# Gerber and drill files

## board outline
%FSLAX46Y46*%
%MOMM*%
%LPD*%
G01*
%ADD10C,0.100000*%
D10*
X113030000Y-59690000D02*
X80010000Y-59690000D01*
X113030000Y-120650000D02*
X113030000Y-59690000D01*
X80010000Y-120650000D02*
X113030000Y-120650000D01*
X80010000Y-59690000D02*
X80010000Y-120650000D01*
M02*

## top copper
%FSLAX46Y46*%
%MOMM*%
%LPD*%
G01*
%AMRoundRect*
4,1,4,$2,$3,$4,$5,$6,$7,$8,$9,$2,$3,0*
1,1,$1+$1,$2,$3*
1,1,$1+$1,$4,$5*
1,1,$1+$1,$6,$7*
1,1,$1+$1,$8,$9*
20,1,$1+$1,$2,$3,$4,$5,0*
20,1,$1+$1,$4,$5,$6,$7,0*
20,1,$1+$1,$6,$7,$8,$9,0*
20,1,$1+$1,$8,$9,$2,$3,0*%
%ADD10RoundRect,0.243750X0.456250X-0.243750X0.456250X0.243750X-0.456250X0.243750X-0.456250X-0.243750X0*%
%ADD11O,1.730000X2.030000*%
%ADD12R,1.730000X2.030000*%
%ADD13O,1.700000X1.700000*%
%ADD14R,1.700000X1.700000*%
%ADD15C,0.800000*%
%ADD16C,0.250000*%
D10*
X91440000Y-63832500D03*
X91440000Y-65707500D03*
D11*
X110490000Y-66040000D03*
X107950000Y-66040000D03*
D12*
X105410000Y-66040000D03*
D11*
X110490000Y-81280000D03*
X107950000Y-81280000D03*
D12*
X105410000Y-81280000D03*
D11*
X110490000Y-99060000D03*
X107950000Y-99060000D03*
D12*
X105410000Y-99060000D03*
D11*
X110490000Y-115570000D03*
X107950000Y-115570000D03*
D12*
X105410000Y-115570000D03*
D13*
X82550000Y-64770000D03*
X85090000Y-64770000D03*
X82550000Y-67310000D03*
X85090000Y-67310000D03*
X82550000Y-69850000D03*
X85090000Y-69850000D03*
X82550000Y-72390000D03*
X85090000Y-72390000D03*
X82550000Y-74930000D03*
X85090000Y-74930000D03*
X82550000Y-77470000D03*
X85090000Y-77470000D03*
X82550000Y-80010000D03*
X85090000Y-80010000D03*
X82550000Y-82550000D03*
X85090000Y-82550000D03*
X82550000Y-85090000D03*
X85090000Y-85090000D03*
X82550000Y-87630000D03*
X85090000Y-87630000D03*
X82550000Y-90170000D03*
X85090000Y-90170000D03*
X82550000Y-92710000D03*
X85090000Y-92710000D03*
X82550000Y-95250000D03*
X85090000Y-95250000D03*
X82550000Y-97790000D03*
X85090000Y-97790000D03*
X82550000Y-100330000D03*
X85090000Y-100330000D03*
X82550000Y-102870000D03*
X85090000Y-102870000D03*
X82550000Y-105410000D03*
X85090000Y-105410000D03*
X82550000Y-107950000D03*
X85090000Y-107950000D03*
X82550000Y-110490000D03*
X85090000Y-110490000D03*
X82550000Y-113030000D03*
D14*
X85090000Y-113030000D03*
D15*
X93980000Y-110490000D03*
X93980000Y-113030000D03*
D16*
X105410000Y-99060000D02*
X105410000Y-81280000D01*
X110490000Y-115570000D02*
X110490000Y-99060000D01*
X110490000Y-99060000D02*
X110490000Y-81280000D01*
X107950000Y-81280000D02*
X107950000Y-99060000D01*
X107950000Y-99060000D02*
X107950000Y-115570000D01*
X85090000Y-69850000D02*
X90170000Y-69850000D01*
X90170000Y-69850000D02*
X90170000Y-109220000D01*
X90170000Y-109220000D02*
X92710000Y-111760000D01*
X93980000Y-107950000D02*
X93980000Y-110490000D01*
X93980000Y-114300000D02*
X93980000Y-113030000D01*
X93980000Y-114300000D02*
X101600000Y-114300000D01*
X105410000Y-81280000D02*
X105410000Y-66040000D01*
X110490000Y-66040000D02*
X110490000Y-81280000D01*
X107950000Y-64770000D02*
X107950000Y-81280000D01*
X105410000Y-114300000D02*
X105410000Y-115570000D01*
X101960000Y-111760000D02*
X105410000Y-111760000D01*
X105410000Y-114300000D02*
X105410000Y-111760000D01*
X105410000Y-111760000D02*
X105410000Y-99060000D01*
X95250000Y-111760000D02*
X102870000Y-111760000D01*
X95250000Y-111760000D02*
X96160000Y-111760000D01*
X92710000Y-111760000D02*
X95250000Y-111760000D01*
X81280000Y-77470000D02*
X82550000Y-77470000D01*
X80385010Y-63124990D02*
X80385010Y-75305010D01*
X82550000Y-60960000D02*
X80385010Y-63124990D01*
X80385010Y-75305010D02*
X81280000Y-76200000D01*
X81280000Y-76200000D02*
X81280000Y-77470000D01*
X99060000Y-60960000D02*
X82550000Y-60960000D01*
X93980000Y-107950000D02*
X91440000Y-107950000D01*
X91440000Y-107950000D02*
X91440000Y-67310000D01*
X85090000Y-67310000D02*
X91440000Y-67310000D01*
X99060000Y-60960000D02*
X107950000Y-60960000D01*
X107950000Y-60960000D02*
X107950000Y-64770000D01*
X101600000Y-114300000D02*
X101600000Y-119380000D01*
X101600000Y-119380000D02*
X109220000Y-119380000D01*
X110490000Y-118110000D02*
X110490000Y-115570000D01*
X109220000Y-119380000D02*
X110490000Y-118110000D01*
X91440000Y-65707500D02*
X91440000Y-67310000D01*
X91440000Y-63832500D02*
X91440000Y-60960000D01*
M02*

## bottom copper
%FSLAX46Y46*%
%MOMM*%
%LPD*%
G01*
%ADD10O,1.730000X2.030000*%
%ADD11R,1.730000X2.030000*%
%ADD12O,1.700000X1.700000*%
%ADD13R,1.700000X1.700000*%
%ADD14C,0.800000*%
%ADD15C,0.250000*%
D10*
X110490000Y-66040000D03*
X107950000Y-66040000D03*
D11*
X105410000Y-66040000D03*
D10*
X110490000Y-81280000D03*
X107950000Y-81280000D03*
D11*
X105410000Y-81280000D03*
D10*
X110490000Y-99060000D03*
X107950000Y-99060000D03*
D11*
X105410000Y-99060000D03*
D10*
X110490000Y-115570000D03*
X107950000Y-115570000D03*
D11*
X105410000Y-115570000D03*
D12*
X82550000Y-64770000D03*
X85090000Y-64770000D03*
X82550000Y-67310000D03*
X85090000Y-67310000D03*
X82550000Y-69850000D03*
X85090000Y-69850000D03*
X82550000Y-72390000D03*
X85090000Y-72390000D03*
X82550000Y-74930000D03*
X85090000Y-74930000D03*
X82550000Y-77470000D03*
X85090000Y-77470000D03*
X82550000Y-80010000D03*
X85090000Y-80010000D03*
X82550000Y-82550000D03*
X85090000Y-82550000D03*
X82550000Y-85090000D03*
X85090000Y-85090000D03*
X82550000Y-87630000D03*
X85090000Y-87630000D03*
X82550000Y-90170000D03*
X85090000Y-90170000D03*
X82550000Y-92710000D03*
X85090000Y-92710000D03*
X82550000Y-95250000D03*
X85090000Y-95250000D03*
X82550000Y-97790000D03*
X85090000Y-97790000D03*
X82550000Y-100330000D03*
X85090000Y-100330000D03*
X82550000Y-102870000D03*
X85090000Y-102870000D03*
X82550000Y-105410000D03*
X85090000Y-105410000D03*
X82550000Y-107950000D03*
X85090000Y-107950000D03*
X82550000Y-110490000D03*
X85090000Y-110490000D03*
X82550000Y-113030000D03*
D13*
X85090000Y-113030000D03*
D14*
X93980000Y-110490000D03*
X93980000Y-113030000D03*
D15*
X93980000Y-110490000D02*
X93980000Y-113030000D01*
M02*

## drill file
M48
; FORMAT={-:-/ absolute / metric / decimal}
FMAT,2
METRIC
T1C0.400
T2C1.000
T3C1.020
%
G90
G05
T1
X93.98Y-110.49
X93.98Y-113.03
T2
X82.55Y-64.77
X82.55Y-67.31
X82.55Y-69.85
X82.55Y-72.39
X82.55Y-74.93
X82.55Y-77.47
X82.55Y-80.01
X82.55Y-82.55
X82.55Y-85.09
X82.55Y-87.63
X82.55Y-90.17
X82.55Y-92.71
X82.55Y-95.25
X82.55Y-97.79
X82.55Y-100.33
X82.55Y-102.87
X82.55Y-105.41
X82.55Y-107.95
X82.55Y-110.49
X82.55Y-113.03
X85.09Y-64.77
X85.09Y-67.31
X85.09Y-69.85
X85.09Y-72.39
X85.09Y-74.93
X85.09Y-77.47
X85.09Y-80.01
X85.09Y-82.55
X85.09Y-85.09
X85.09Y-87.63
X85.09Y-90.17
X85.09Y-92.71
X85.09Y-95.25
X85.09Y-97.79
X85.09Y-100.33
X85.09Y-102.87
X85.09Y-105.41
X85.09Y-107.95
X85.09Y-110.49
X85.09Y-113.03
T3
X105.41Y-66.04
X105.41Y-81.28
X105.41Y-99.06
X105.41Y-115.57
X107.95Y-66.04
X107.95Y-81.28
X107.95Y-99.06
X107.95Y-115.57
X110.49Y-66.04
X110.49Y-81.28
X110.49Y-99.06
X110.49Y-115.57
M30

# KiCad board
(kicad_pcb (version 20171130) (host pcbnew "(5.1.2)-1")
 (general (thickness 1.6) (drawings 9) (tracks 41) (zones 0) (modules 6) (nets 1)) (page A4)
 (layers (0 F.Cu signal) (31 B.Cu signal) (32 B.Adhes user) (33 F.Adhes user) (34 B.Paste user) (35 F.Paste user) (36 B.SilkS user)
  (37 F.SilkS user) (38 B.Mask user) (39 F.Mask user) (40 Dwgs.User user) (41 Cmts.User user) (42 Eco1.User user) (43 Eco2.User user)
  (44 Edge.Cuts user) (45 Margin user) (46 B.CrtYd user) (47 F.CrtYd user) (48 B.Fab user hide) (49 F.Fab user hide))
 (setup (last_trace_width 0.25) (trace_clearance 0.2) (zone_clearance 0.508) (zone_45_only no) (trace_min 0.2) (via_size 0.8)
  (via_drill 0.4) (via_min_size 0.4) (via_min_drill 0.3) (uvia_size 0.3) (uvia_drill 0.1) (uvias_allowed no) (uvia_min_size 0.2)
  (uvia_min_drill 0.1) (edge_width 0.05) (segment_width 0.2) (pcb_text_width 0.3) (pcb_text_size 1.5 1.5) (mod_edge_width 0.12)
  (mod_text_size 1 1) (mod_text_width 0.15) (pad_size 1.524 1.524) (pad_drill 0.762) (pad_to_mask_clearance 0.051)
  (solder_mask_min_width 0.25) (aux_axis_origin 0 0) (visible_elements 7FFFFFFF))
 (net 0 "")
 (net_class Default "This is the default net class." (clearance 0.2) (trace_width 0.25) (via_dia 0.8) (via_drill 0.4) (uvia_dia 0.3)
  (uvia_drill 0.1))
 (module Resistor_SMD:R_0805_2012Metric (layer F.Cu) (at 91.44 64.77 90)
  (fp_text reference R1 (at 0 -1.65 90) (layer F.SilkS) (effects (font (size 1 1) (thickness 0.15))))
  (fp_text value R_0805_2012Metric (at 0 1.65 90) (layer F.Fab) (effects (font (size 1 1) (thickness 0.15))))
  (pad 2 smd roundrect (at 0.9375 0 90) (size 0.975 1.4) (layers F.Cu F.Paste F.Mask) (roundrect_rratio 0.25))
  (pad 1 smd roundrect (at -0.9375 0 90) (size 0.975 1.4) (layers F.Cu F.Paste F.Mask) (roundrect_rratio 0.25)))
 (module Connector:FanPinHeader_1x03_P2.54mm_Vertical (layer F.Cu) (at 105.41 66.04)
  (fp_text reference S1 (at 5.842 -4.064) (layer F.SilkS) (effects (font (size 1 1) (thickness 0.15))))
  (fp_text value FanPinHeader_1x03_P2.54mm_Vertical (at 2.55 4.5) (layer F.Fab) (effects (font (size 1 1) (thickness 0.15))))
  (pad 3 thru_hole oval (at 5.08 0 90) (size 2.03 1.73) (drill 1.02) (layers *.Cu *.Mask))
  (pad 2 thru_hole oval (at 2.54 0 90) (size 2.03 1.73) (drill 1.02) (layers *.Cu *.Mask))
  (pad 1 thru_hole rect (at 0 0 90) (size 2.03 1.73) (drill 1.02) (layers *.Cu *.Mask)))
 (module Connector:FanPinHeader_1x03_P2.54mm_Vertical (layer F.Cu) (at 105.41 81.28)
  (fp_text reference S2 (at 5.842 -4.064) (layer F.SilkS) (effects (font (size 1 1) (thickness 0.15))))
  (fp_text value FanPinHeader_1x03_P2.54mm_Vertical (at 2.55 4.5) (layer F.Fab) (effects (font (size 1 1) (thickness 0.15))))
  (pad 3 thru_hole oval (at 5.08 0 90) (size 2.03 1.73) (drill 1.02) (layers *.Cu *.Mask))
  (pad 2 thru_hole oval (at 2.54 0 90) (size 2.03 1.73) (drill 1.02) (layers *.Cu *.Mask))
  (pad 1 thru_hole rect (at 0 0 90) (size 2.03 1.73) (drill 1.02) (layers *.Cu *.Mask)))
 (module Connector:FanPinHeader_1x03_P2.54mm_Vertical (layer F.Cu) (at 105.41 99.06)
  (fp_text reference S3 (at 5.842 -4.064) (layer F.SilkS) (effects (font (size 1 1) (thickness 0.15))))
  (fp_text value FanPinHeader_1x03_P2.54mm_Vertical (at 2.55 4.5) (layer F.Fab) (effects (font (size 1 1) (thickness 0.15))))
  (pad 3 thru_hole oval (at 5.08 0 90) (size 2.03 1.73) (drill 1.02) (layers *.Cu *.Mask))
  (pad 2 thru_hole oval (at 2.54 0 90) (size 2.03 1.73) (drill 1.02) (layers *.Cu *.Mask))
  (pad 1 thru_hole rect (at 0 0 90) (size 2.03 1.73) (drill 1.02) (layers *.Cu *.Mask)))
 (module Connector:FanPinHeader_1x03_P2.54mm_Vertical (layer F.Cu) (at 105.41 115.57)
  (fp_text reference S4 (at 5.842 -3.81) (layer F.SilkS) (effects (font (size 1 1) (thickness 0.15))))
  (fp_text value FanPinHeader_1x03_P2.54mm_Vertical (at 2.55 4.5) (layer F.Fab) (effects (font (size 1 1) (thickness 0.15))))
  (pad 3 thru_hole oval (at 5.08 0 90) (size 2.03 1.73) (drill 1.02) (layers *.Cu *.Mask))
  (pad 2 thru_hole oval (at 2.54 0 90) (size 2.03 1.73) (drill 1.02) (layers *.Cu *.Mask))
  (pad 1 thru_hole rect (at 0 0 90) (size 2.03 1.73) (drill 1.02) (layers *.Cu *.Mask)))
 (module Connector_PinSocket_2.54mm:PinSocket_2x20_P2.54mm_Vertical (layer B.Cu) (at 85.09 113.03)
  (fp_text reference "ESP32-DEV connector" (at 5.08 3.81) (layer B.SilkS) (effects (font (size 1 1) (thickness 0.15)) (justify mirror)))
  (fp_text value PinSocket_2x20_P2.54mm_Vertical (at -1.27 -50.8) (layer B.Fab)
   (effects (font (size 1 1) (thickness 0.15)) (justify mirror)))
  (pad 40 thru_hole oval (at -2.54 -48.26) (size 1.7 1.7) (drill 1) (layers *.Cu *.Mask))
  (pad 39 thru_hole oval (at 0 -48.26) (size 1.7 1.7) (drill 1) (layers *.Cu *.Mask))
  (pad 38 thru_hole oval (at -2.54 -45.72) (size 1.7 1.7) (drill 1) (layers *.Cu *.Mask))
  (pad 37 thru_hole oval (at 0 -45.72) (size 1.7 1.7) (drill 1) (layers *.Cu *.Mask))
  (pad 36 thru_hole oval (at -2.54 -43.18) (size 1.7 1.7) (drill 1) (layers *.Cu *.Mask))
  (pad 35 thru_hole oval (at 0 -43.18) (size 1.7 1.7) (drill 1) (layers *.Cu *.Mask))
  (pad 34 thru_hole oval (at -2.54 -40.64) (size 1.7 1.7) (drill 1) (layers *.Cu *.Mask))
  (pad 33 thru_hole oval (at 0 -40.64) (size 1.7 1.7) (drill 1) (layers *.Cu *.Mask))
  (pad 32 thru_hole oval (at -2.54 -38.1) (size 1.7 1.7) (drill 1) (layers *.Cu *.Mask))
  (pad 31 thru_hole oval (at 0 -38.1) (size 1.7 1.7) (drill 1) (layers *.Cu *.Mask))
  (pad 30 thru_hole oval (at -2.54 -35.56) (size 1.7 1.7) (drill 1) (layers *.Cu *.Mask))
  (pad 29 thru_hole oval (at 0 -35.56) (size 1.7 1.7) (drill 1) (layers *.Cu *.Mask))
  (pad 28 thru_hole oval (at -2.54 -33.02) (size 1.7 1.7) (drill 1) (layers *.Cu *.Mask))
  (pad 27 thru_hole oval (at 0 -33.02) (size 1.7 1.7) (drill 1) (layers *.Cu *.Mask))
  (pad 26 thru_hole oval (at -2.54 -30.48) (size 1.7 1.7) (drill 1) (layers *.Cu *.Mask))
  (pad 25 thru_hole oval (at 0 -30.48) (size 1.7 1.7) (drill 1) (layers *.Cu *.Mask))
  (pad 24 thru_hole oval (at -2.54 -27.94) (size 1.7 1.7) (drill 1) (layers *.Cu *.Mask))
  (pad 23 thru_hole oval (at 0 -27.94) (size 1.7 1.7) (drill 1) (layers *.Cu *.Mask))
  (pad 22 thru_hole oval (at -2.54 -25.4) (size 1.7 1.7) (drill 1) (layers *.Cu *.Mask))
  (pad 21 thru_hole oval (at 0 -25.4) (size 1.7 1.7) (drill 1) (layers *.Cu *.Mask))
  (pad 20 thru_hole oval (at -2.54 -22.86) (size 1.7 1.7) (drill 1) (layers *.Cu *.Mask))
  (pad 19 thru_hole oval (at 0 -22.86) (size 1.7 1.7) (drill 1) (layers *.Cu *.Mask))
  (pad 18 thru_hole oval (at -2.54 -20.32) (size 1.7 1.7) (drill 1) (layers *.Cu *.Mask))
  (pad 17 thru_hole oval (at 0 -20.32) (size 1.7 1.7) (drill 1) (layers *.Cu *.Mask))
  (pad 16 thru_hole oval (at -2.54 -17.78) (size 1.7 1.7) (drill 1) (layers *.Cu *.Mask))
  (pad 15 thru_hole oval (at 0 -17.78) (size 1.7 1.7) (drill 1) (layers *.Cu *.Mask))
  (pad 14 thru_hole oval (at -2.54 -15.24) (size 1.7 1.7) (drill 1) (layers *.Cu *.Mask))
  (pad 13 thru_hole oval (at 0 -15.24) (size 1.7 1.7) (drill 1) (layers *.Cu *.Mask))
  (pad 12 thru_hole oval (at -2.54 -12.7) (size 1.7 1.7) (drill 1) (layers *.Cu *.Mask))
  (pad 11 thru_hole oval (at 0 -12.7) (size 1.7 1.7) (drill 1) (layers *.Cu *.Mask))
  (pad 10 thru_hole oval (at -2.54 -10.16) (size 1.7 1.7) (drill 1) (layers *.Cu *.Mask))
  (pad 9 thru_hole oval (at 0 -10.16) (size 1.7 1.7) (drill 1) (layers *.Cu *.Mask))
  (pad 8 thru_hole oval (at -2.54 -7.62) (size 1.7 1.7) (drill 1) (layers *.Cu *.Mask))
  (pad 7 thru_hole oval (at 0 -7.62) (size 1.7 1.7) (drill 1) (layers *.Cu *.Mask))
  (pad 6 thru_hole oval (at -2.54 -5.08) (size 1.7 1.7) (drill 1) (layers *.Cu *.Mask))
  (pad 5 thru_hole oval (at 0 -5.08) (size 1.7 1.7) (drill 1) (layers *.Cu *.Mask))
  (pad 4 thru_hole oval (at -2.54 -2.54) (size 1.7 1.7) (drill 1) (layers *.Cu *.Mask))
  (pad 3 thru_hole oval (at 0 -2.54) (size 1.7 1.7) (drill 1) (layers *.Cu *.Mask))
  (pad 2 thru_hole oval (at -2.54 0) (size 1.7 1.7) (drill 1) (layers *.Cu *.Mask))
  (pad 1 thru_hole rect (at 0 0) (size 1.7 1.7) (drill 1) (layers *.Cu *.Mask)))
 (gr_line (start 113.03 59.69) (end 80.01 59.69) (layer Edge.Cuts) (width 0.1))
 (gr_line (start 113.03 120.65) (end 113.03 59.69) (layer Edge.Cuts) (width 0.1))
 (gr_line (start 80.01 120.65) (end 113.03 120.65) (layer Edge.Cuts) (width 0.1))
 (gr_line (start 80.01 59.69) (end 80.01 120.65) (layer Edge.Cuts) (width 0.1))
 (segment (start 105.41 99.06) (end 105.41 81.28) (width 0.25) (layer F.Cu) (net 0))
 (segment (start 110.49 115.57) (end 110.49 99.06) (width 0.25) (layer F.Cu) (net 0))
 (segment (start 110.49 99.06) (end 110.49 81.28) (width 0.25) (layer F.Cu) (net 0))
 (segment (start 107.95 81.28) (end 107.95 99.06) (width 0.25) (layer F.Cu) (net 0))
 (segment (start 107.95 99.06) (end 107.95 115.57) (width 0.25) (layer F.Cu) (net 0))
 (segment (start 85.09 69.85) (end 90.17 69.85) (width 0.25) (layer F.Cu) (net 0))
 (segment (start 90.17 69.85) (end 90.17 109.22) (width 0.25) (layer F.Cu) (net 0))
 (segment (start 90.17 109.22) (end 92.71 111.76) (width 0.25) (layer F.Cu) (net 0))
 (segment (start 93.98 107.95) (end 93.98 110.49) (width 0.25) (layer F.Cu) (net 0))
 (via (at 93.98 110.49) (size 0.8) (drill 0.4) (layers F.Cu B.Cu) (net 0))
 (segment (start 93.98 114.3) (end 93.98 113.03) (width 0.25) (layer F.Cu) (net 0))
 (via (at 93.98 113.03) (size 0.8) (drill 0.4) (layers F.Cu B.Cu) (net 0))
 (segment (start 93.98 114.3) (end 101.6 114.3) (width 0.25) (layer F.Cu) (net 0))
 (segment (start 93.98 110.49) (end 93.98 113.03) (width 0.25) (layer B.Cu) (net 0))
 (segment (start 105.41 81.28) (end 105.41 66.04) (width 0.25) (layer F.Cu) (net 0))
 (segment (start 110.49 66.04) (end 110.49 81.28) (width 0.25) (layer F.Cu) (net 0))
 (segment (start 107.95 64.77) (end 107.95 81.28) (width 0.25) (layer F.Cu) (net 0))
 (segment (start 105.41 114.3) (end 105.41 115.57) (width 0.25) (layer F.Cu) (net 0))
 (segment (start 101.96 111.76) (end 105.41 111.76) (width 0.25) (layer F.Cu) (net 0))
 (segment (start 105.41 114.3) (end 105.41 111.76) (width 0.25) (layer F.Cu) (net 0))
 (segment (start 105.41 111.76) (end 105.41 99.06) (width 0.25) (layer F.Cu) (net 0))
 (segment (start 95.25 111.76) (end 102.87 111.76) (width 0.25) (layer F.Cu) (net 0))
 (segment (start 95.25 111.76) (end 96.16 111.76) (width 0.25) (layer F.Cu) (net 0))
 (segment (start 92.71 111.76) (end 95.25 111.76) (width 0.25) (layer F.Cu) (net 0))
 (segment (start 81.28 77.47) (end 82.55 77.47) (width 0.25) (layer F.Cu) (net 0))
 (segment (start 80.38501 63.12499) (end 80.38501 75.30501) (width 0.25) (layer F.Cu) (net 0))
 (segment (start 82.55 60.96) (end 80.38501 63.12499) (width 0.25) (layer F.Cu) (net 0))
 (segment (start 80.38501 75.30501) (end 81.28 76.2) (width 0.25) (layer F.Cu) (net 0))
 (segment (start 81.28 76.2) (end 81.28 77.47) (width 0.25) (layer F.Cu) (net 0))
 (segment (start 99.06 60.96) (end 82.55 60.96) (width 0.25) (layer F.Cu) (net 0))
 (segment (start 93.98 107.95) (end 91.44 107.95) (width 0.25) (layer F.Cu) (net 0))
 (segment (start 91.44 107.95) (end 91.44 67.31) (width 0.25) (layer F.Cu) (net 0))
 (segment (start 85.09 67.31) (end 91.44 67.31) (width 0.25) (layer F.Cu) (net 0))
 (segment (start 99.06 60.96) (end 107.95 60.96) (width 0.25) (layer F.Cu) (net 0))
 (segment (start 107.95 60.96) (end 107.95 64.77) (width 0.25) (layer F.Cu) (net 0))
 (segment (start 101.6 114.3) (end 101.6 119.38) (width 0.25) (layer F.Cu) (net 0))
 (segment (start 101.6 119.38) (end 109.22 119.38) (width 0.25) (layer F.Cu) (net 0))
 (segment (start 110.49 118.11) (end 110.49 115.57) (width 0.25) (layer F.Cu) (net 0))
 (segment (start 109.22 119.38) (end 110.49 118.11) (width 0.25) (layer F.Cu) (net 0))
 (segment (start 91.44 65.7075) (end 91.44 67.31) (width 0.25) (layer F.Cu) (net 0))
 (segment (start 91.44 63.8325) (end 91.44 60.96) (width 0.25) (layer F.Cu) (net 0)))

